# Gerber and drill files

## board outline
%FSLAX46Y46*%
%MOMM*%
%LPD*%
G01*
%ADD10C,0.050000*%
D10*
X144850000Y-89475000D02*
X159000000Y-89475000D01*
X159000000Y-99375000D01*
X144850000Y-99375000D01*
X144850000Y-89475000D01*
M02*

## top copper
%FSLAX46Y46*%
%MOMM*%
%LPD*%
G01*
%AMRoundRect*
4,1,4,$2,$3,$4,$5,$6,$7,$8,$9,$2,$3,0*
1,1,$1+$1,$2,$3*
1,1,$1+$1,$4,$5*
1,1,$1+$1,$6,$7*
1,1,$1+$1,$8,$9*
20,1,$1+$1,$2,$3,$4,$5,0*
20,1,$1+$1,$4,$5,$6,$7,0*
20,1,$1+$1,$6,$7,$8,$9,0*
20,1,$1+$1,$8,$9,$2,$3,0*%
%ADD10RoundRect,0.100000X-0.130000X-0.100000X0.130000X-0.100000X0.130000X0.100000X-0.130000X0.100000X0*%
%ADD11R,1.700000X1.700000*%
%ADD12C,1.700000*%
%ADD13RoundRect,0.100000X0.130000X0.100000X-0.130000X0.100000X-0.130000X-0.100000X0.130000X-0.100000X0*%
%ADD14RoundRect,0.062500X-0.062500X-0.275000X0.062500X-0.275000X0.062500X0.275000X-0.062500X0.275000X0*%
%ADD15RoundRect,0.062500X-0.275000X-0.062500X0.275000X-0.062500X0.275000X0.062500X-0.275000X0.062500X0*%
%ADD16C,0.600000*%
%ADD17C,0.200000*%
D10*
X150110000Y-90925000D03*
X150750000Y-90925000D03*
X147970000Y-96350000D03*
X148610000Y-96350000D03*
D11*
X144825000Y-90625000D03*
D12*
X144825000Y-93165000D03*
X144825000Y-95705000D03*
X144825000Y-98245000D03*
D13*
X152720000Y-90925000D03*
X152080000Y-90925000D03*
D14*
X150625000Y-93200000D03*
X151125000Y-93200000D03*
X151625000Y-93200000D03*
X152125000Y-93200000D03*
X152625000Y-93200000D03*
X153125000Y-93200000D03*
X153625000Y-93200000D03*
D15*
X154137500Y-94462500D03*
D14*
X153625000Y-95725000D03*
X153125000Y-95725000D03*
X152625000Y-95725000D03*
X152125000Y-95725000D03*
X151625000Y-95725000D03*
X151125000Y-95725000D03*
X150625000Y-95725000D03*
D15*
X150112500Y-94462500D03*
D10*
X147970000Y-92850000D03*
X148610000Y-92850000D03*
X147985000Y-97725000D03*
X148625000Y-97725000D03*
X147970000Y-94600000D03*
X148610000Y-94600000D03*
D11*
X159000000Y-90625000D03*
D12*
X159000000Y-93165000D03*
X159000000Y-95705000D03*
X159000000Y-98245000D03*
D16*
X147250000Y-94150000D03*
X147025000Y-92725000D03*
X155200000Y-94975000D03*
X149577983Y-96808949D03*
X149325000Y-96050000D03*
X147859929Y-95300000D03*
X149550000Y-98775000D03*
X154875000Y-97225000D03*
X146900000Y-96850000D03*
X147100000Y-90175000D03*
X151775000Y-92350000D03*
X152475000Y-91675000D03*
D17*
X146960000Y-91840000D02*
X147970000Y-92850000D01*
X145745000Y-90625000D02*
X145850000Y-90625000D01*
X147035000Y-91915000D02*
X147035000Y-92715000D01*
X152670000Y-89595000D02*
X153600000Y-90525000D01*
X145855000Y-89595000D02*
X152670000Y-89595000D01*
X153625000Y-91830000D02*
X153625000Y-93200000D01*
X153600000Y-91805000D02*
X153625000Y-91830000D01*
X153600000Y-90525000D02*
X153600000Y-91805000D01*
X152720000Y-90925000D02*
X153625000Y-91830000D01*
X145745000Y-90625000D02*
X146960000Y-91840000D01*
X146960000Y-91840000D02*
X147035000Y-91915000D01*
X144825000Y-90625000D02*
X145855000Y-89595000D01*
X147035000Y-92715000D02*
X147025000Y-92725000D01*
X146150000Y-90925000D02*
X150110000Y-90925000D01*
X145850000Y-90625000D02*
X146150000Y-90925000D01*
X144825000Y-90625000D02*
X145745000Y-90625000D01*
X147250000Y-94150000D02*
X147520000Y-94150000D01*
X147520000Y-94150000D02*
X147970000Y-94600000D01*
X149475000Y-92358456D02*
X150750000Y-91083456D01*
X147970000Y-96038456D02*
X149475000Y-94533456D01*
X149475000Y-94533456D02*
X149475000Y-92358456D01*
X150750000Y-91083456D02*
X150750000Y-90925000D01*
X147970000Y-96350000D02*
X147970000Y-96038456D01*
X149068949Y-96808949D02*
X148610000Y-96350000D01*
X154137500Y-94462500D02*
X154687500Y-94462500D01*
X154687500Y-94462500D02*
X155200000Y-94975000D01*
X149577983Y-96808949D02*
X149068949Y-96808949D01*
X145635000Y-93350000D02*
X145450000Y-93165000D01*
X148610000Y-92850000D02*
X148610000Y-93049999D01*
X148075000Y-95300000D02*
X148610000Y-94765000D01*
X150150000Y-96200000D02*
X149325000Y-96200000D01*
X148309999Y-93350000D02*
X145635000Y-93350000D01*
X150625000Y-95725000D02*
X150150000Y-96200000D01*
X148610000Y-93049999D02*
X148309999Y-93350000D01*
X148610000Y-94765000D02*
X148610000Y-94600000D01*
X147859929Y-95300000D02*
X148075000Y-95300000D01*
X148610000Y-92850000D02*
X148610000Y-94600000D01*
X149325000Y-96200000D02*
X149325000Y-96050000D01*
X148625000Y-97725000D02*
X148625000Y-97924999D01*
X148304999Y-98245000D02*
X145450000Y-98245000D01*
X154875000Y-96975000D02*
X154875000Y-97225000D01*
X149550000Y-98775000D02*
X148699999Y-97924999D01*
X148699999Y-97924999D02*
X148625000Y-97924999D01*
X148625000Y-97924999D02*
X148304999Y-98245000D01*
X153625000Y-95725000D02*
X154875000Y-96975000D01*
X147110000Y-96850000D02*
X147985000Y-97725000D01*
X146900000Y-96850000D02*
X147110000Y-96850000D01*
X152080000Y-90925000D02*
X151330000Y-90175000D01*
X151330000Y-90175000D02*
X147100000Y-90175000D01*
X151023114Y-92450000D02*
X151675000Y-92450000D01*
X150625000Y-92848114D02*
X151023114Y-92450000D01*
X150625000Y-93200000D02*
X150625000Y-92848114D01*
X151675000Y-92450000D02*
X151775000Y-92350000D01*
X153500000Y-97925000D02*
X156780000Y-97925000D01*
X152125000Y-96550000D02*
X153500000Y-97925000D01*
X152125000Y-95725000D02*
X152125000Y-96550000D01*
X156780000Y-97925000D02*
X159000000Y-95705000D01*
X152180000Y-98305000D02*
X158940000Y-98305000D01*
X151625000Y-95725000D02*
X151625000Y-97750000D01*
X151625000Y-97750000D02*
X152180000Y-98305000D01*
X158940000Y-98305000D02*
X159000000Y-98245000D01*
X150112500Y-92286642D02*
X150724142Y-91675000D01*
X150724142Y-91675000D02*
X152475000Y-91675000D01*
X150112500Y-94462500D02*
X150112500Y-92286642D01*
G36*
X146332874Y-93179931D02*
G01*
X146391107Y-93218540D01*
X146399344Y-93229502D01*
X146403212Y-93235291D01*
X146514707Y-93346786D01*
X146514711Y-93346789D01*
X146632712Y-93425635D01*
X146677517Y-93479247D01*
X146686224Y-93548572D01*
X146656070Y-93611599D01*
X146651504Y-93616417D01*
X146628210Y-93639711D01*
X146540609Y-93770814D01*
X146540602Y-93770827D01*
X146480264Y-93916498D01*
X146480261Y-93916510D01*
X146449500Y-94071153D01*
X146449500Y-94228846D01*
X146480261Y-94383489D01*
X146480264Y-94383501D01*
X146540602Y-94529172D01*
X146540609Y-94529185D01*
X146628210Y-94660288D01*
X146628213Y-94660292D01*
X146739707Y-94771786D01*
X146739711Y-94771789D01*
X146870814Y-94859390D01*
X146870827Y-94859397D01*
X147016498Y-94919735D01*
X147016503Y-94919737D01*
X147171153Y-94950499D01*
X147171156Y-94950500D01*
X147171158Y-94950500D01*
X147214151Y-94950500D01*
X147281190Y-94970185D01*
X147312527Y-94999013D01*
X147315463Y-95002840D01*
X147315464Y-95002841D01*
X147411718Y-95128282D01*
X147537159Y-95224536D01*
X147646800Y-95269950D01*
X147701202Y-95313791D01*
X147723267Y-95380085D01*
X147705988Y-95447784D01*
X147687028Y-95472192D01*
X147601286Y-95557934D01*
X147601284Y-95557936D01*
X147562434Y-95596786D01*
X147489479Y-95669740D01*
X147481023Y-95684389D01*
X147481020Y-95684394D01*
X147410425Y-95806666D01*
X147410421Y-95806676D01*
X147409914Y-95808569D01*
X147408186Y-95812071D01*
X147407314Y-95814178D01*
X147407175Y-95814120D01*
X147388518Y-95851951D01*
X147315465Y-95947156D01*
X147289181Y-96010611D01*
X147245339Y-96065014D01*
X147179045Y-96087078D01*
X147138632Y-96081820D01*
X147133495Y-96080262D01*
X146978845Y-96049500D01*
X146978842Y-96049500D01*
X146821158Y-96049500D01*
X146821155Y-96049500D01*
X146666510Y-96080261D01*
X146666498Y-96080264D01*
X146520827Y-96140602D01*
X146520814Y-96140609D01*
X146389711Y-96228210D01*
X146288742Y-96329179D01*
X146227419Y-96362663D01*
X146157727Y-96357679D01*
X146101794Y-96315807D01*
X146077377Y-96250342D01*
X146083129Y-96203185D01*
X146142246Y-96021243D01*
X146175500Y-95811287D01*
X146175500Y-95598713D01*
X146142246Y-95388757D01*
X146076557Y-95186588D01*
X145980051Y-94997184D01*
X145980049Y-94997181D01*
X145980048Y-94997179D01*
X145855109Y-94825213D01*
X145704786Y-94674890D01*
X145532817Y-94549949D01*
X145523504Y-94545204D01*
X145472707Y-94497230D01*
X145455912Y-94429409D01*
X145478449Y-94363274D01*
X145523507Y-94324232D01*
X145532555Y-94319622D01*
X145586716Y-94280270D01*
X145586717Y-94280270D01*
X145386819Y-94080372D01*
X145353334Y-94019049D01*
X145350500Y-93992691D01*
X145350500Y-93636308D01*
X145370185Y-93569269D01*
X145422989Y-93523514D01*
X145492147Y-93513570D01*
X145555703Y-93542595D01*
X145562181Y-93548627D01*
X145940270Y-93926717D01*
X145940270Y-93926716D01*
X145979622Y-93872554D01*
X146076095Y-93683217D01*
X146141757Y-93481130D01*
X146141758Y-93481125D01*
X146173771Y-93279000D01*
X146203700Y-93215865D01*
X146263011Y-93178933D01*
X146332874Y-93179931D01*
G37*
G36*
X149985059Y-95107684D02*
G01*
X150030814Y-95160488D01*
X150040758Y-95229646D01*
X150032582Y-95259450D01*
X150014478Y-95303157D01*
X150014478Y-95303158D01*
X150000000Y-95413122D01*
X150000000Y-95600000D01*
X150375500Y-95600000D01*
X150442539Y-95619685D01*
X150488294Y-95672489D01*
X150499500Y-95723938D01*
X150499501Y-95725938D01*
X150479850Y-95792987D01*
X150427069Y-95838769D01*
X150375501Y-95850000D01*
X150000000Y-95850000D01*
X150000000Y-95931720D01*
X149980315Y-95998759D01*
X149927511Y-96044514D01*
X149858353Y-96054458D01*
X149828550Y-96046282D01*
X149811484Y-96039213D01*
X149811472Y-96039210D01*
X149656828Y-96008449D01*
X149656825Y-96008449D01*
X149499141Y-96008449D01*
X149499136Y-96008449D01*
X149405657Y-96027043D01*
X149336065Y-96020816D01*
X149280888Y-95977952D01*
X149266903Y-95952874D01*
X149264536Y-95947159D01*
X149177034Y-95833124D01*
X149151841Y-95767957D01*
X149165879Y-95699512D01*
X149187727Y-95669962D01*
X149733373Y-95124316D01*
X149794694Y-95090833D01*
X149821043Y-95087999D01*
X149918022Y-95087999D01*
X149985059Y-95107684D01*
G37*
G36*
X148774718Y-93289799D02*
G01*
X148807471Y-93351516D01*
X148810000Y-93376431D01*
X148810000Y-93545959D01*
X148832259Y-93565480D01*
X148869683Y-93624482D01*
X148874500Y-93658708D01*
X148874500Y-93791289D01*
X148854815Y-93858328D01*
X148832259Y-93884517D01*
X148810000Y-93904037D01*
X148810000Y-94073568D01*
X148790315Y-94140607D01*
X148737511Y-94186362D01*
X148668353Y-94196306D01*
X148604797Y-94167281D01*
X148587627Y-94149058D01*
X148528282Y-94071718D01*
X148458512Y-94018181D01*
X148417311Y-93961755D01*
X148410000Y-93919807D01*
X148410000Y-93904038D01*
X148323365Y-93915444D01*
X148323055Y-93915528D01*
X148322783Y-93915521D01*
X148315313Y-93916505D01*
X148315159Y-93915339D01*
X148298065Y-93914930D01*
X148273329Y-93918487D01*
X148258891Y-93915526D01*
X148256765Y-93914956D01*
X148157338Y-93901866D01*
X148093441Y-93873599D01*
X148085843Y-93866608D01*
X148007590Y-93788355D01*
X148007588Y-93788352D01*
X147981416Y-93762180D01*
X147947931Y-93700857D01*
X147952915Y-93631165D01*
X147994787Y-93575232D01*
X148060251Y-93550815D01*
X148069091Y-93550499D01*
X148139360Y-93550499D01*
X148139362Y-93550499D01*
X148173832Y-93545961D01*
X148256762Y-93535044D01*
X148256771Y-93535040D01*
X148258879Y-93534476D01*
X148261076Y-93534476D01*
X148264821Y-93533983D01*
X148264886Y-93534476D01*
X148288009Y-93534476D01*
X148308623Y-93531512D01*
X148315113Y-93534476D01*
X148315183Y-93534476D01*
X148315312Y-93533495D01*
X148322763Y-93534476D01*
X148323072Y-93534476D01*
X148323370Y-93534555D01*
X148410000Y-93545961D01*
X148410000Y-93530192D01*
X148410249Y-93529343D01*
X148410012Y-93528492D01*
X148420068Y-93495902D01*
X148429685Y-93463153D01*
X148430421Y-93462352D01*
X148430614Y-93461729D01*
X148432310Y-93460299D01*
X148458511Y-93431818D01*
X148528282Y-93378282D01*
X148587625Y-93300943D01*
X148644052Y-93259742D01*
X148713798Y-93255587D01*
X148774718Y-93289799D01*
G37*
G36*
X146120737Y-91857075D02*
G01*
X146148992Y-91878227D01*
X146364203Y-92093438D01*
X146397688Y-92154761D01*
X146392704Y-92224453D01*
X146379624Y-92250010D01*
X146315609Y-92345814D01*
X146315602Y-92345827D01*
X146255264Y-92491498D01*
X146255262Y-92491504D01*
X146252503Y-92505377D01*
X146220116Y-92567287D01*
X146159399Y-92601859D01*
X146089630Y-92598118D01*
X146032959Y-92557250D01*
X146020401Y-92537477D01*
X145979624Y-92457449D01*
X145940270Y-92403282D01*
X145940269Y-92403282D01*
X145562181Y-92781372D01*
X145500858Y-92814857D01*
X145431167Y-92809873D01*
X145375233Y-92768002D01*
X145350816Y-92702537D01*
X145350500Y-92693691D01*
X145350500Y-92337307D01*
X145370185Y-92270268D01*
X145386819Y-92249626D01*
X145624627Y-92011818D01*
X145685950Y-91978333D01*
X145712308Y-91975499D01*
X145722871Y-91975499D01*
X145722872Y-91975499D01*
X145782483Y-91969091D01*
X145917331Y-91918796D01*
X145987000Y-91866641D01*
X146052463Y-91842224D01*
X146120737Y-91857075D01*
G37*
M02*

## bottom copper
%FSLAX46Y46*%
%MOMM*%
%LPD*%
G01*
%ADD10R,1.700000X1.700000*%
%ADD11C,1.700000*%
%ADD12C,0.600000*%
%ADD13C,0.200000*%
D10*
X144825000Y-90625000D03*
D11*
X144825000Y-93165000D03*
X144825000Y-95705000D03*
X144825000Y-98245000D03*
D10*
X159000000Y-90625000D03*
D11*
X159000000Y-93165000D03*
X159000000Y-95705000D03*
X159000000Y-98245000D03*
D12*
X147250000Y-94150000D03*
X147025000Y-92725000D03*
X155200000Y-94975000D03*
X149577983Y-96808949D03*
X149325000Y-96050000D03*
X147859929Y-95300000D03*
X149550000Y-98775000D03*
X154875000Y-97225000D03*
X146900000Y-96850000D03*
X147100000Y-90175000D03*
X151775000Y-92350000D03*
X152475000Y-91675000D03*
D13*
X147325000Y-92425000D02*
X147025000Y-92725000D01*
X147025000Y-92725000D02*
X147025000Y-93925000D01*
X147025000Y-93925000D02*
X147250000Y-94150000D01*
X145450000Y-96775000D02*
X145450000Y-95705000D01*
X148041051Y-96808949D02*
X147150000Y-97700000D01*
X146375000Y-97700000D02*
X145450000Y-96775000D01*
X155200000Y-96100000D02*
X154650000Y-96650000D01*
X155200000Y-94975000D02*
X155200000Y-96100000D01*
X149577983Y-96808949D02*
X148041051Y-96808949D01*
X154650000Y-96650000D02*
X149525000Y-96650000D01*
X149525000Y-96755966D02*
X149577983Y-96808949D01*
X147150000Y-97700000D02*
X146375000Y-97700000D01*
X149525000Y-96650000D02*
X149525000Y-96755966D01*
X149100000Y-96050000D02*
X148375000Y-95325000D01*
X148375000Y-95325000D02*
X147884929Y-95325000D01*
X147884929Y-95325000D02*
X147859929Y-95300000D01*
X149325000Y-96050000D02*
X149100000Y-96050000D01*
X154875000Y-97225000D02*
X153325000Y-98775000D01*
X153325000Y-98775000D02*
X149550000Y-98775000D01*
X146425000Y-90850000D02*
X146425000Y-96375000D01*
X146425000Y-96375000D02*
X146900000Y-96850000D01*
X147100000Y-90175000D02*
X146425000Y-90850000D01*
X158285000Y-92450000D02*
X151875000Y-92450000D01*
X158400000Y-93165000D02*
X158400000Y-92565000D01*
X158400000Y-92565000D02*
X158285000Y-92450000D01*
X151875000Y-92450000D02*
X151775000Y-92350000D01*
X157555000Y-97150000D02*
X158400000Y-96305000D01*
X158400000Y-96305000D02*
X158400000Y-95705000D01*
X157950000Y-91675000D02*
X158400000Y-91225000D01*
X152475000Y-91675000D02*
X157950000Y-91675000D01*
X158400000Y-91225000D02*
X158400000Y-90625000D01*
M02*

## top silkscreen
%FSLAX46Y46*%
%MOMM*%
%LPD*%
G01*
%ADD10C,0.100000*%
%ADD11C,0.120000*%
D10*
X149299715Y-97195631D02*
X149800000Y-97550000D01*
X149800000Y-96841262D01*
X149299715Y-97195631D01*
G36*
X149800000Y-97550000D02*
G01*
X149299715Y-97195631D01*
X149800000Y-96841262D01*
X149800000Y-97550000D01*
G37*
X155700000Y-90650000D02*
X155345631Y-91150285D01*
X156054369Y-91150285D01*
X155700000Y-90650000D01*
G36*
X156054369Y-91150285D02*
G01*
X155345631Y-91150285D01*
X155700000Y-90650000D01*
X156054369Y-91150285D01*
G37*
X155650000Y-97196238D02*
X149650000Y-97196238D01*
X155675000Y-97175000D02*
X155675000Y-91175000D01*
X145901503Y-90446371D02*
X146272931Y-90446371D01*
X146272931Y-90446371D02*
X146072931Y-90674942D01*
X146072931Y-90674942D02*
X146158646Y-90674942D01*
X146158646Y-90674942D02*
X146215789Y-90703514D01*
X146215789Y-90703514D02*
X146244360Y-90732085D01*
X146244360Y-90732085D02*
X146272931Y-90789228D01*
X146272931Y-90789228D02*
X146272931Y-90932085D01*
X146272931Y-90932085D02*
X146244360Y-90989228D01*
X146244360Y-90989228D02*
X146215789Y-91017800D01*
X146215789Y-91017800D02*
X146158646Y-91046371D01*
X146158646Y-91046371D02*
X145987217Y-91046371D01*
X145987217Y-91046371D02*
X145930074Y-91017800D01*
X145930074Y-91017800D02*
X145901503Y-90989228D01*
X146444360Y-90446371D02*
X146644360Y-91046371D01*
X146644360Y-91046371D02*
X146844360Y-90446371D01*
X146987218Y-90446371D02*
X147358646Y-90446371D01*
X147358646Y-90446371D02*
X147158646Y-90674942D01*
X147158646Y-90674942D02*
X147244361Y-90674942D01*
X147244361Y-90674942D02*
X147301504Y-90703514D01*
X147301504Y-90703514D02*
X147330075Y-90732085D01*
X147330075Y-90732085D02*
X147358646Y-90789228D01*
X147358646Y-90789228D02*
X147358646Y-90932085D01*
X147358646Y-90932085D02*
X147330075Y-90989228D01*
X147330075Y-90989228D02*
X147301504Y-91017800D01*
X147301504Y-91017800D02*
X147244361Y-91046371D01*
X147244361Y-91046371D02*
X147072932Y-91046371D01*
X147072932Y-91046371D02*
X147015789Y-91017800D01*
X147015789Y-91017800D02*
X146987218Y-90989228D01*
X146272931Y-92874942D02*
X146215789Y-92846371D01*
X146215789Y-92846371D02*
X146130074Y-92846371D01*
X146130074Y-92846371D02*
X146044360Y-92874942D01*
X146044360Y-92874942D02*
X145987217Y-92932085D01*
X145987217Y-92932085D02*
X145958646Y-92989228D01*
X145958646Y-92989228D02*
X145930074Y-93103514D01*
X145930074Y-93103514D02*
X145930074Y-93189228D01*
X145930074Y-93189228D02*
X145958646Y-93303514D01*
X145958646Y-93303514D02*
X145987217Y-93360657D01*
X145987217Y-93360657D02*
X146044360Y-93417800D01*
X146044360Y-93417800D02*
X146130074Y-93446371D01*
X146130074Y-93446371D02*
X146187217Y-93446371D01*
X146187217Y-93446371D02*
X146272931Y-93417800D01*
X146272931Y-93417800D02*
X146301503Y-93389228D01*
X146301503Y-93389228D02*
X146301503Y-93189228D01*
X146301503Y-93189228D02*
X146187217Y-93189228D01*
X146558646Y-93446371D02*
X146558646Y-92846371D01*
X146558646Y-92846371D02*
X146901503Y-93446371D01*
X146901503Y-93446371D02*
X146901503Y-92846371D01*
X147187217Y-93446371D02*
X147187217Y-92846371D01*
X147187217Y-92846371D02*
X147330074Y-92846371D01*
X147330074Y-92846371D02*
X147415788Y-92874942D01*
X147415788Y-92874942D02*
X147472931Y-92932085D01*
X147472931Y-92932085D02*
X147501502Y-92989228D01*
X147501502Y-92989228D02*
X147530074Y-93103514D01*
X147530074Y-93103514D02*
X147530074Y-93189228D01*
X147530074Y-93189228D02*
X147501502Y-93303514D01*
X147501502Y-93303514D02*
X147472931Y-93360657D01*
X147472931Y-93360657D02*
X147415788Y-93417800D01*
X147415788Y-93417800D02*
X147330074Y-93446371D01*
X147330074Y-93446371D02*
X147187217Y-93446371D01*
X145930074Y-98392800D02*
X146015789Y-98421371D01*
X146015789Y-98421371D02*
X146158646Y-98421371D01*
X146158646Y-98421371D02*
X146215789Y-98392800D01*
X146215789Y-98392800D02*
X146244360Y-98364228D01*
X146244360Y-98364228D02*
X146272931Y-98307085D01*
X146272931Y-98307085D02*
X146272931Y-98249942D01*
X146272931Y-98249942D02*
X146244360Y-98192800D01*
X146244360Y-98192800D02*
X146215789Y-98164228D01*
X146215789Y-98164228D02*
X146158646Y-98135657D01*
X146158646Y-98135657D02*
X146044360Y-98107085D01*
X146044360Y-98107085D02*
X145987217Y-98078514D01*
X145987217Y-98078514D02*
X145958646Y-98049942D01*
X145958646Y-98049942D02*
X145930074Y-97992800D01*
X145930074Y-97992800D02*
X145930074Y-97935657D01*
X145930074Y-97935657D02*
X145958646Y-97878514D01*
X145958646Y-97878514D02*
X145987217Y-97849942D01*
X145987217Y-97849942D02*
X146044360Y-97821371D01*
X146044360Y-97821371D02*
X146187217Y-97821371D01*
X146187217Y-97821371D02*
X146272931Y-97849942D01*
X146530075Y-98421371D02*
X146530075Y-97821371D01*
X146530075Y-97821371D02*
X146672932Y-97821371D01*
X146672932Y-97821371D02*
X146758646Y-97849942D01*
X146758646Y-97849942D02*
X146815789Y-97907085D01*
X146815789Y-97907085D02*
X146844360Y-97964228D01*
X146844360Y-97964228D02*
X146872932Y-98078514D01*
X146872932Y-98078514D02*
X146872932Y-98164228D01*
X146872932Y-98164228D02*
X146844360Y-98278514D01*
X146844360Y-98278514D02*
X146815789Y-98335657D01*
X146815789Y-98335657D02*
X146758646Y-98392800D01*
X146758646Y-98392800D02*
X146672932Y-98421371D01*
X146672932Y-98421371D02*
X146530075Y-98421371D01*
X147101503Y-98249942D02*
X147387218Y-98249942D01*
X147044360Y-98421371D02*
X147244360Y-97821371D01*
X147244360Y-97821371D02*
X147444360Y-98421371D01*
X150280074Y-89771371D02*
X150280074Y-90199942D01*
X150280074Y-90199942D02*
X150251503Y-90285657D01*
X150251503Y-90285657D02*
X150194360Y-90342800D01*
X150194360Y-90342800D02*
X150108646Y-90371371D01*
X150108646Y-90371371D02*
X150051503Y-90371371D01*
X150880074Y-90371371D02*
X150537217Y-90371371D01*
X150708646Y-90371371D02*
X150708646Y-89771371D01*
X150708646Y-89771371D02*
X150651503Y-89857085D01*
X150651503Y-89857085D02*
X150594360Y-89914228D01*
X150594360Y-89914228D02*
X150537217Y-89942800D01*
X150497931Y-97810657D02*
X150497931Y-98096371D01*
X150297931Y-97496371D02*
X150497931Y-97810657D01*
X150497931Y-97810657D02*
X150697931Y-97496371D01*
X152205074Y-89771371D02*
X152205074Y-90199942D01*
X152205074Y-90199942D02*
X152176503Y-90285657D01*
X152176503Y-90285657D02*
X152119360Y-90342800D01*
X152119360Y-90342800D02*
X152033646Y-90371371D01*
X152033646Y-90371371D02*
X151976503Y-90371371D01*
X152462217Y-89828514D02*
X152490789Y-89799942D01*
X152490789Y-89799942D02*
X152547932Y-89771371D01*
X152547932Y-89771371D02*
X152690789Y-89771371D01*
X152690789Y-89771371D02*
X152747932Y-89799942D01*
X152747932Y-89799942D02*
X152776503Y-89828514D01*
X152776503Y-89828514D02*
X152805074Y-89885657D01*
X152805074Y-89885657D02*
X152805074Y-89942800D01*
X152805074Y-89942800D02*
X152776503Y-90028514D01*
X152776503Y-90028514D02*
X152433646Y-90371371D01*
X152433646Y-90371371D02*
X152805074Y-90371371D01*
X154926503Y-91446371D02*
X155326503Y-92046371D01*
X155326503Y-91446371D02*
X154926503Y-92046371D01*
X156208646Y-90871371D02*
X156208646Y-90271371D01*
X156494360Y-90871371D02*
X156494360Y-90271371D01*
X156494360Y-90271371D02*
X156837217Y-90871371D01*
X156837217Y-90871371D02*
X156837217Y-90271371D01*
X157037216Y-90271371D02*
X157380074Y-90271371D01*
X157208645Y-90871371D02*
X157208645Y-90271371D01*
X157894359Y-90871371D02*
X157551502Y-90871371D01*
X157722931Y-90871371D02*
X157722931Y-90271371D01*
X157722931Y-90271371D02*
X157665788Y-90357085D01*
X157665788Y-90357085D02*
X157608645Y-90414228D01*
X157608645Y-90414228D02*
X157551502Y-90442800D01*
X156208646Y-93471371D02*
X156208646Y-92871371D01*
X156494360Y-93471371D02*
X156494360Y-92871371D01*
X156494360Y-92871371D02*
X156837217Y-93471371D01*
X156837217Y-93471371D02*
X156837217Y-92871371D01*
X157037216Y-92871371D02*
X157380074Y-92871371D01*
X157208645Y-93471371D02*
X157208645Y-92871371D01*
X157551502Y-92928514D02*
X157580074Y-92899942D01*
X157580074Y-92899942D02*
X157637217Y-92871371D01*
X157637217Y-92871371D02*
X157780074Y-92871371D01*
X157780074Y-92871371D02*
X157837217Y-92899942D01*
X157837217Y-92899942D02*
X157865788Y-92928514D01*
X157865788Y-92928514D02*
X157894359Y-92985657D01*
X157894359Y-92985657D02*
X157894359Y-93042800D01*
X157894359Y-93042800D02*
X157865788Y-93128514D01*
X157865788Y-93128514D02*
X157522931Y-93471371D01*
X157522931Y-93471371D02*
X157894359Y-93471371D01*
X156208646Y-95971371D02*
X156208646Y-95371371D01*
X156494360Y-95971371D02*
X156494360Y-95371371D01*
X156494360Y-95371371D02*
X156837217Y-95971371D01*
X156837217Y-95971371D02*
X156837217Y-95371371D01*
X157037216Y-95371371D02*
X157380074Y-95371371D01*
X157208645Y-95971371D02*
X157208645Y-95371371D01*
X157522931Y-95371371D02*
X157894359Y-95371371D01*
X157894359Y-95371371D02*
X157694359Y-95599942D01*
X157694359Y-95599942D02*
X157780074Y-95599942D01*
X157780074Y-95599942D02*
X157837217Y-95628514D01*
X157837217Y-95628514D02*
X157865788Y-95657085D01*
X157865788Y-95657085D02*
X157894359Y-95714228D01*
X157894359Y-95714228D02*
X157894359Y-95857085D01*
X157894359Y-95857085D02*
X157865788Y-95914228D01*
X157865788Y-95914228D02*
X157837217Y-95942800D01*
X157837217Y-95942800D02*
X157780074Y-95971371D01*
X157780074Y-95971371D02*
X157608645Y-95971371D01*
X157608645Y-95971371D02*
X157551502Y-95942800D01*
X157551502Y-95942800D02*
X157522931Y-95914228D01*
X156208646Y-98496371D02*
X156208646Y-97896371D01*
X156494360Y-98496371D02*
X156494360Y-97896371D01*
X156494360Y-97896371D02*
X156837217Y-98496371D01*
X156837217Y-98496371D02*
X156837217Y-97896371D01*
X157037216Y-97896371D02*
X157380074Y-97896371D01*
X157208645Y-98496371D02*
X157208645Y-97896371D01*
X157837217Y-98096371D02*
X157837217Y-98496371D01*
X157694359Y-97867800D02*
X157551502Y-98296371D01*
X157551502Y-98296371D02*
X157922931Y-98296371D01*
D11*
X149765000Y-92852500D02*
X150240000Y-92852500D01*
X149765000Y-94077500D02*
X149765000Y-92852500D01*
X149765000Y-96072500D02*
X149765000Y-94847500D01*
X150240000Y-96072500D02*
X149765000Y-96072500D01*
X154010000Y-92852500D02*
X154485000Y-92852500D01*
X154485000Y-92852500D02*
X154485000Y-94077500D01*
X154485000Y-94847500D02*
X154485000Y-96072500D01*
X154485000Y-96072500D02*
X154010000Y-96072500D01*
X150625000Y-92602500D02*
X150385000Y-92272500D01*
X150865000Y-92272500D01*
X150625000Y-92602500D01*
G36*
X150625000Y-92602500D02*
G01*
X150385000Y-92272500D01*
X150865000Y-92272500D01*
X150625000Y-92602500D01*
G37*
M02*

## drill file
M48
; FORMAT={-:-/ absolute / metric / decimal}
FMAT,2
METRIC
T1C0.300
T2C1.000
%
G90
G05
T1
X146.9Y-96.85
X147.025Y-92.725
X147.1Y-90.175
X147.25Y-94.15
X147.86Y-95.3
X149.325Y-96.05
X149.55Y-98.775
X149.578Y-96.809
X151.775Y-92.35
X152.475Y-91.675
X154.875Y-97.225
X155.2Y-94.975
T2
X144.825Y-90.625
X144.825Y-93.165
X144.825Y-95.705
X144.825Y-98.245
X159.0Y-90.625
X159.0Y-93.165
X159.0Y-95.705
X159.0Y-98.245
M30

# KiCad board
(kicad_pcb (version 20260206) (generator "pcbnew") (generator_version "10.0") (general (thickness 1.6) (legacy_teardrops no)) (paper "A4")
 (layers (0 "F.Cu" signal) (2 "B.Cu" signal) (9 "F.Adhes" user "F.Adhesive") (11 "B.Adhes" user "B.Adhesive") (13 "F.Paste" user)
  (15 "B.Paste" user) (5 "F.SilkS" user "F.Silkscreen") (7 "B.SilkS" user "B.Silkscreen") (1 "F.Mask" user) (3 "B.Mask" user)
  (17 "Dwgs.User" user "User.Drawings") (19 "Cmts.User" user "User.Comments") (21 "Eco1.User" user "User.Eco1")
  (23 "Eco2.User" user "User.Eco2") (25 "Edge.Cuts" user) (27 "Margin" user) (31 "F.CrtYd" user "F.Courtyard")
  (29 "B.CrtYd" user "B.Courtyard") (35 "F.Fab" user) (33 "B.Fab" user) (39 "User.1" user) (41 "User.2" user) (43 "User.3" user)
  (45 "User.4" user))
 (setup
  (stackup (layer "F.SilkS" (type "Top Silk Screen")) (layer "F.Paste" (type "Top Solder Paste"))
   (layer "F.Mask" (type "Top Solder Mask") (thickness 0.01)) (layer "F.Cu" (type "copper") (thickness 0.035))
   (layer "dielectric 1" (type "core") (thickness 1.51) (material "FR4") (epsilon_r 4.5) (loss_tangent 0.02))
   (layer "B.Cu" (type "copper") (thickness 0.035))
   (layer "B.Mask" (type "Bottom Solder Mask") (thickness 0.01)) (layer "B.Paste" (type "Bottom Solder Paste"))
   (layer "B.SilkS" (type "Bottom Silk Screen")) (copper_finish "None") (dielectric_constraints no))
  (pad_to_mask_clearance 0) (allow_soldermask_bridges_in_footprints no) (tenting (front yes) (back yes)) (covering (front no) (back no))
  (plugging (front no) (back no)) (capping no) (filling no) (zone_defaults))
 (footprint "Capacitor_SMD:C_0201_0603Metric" (layer "F.Cu") (at 150.43 90.925)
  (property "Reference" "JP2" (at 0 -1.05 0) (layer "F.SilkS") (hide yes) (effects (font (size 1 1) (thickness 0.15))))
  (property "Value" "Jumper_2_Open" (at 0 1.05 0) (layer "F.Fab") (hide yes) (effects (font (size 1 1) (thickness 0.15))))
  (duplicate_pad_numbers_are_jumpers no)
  (pad "" smd roundrect (at -0.345 0) (size 0.318 0.36) (layers "F.Paste") (roundrect_rratio 0.25))
  (pad "" smd roundrect (at 0.345 0) (size 0.318 0.36) (layers "F.Paste") (roundrect_rratio 0.25))
  (pad "1" smd roundrect (at -0.32 0) (size 0.46 0.4) (layers "F.Cu" "F.Mask") (roundrect_rratio 0.25) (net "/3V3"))
  (pad "2" smd roundrect (at 0.32 0) (size 0.46 0.4) (layers "F.Cu" "F.Mask") (roundrect_rratio 0.25) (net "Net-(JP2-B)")))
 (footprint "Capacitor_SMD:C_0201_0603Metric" (layer "F.Cu") (at 148.29 96.35)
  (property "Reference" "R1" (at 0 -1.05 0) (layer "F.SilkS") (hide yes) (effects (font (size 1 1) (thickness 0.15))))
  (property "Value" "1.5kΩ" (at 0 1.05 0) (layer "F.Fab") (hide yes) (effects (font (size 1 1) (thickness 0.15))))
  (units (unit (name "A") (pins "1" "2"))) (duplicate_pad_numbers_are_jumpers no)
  (pad "" smd roundrect (at -0.345 0) (size 0.318 0.36) (layers "F.Paste") (roundrect_rratio 0.25))
  (pad "" smd roundrect (at 0.345 0) (size 0.318 0.36) (layers "F.Paste") (roundrect_rratio 0.25))
  (pad "1" smd roundrect (at -0.32 0) (size 0.46 0.4) (layers "F.Cu" "F.Mask") (roundrect_rratio 0.25) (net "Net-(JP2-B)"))
  (pad "2" smd roundrect (at 0.32 0) (size 0.46 0.4) (layers "F.Cu" "F.Mask") (roundrect_rratio 0.25) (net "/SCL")))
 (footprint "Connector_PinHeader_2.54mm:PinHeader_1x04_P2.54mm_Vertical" (layer "F.Cu") (at 144.825 90.625)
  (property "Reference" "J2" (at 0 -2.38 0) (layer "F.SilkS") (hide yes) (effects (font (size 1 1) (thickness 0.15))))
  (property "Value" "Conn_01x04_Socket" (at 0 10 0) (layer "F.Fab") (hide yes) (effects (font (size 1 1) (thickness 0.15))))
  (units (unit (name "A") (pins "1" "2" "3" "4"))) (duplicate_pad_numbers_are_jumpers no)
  (pad "1" thru_hole rect (at 0 0) (size 1.7 1.7) (drill 1) (layers "*.Cu" "*.Mask") (remove_unused_layers no) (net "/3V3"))
  (pad "2" thru_hole circle (at 0 2.54) (size 1.7 1.7) (drill 1) (layers "*.Cu" "*.Mask") (remove_unused_layers no) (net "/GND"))
  (pad "3" thru_hole circle (at 0 5.08) (size 1.7 1.7) (drill 1) (layers "*.Cu" "*.Mask") (remove_unused_layers no) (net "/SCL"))
  (pad "4" thru_hole circle (at 0 7.62) (size 1.7 1.7) (drill 1) (layers "*.Cu" "*.Mask") (remove_unused_layers no) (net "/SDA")))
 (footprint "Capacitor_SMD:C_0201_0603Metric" (layer "F.Cu") (at 152.4 90.925 180)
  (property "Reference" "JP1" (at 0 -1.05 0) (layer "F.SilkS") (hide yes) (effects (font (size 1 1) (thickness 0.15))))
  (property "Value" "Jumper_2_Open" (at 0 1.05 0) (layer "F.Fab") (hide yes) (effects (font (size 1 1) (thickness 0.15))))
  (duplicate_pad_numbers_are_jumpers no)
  (pad "" smd roundrect (at -0.345 0 180) (size 0.318 0.36) (layers "F.Paste") (roundrect_rratio 0.25))
  (pad "" smd roundrect (at 0.345 0 180) (size 0.318 0.36) (layers "F.Paste") (roundrect_rratio 0.25))
  (pad "1" smd roundrect (at -0.32 0 180) (size 0.46 0.4) (layers "F.Cu" "F.Mask") (roundrect_rratio 0.25) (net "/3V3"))
  (pad "2" smd roundrect (at 0.32 0 180) (size 0.46 0.4) (layers "F.Cu" "F.Mask") (roundrect_rratio 0.25) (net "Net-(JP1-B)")))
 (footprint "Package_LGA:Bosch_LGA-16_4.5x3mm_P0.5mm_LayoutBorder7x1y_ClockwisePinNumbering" (layer "F.Cu") (at 152.125 94.4625)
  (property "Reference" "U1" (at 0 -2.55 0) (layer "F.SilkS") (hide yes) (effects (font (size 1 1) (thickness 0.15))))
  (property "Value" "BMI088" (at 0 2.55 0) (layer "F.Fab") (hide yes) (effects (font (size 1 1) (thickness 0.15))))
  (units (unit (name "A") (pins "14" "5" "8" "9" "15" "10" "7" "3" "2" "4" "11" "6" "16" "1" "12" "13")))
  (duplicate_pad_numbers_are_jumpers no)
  (fp_line (start -2.36 -1.61) (end -1.885 -1.61) (stroke (width 0.12) (type solid)) (layer "F.SilkS"))
  (fp_line (start -2.36 -0.385) (end -2.36 -1.61) (stroke (width 0.12) (type solid)) (layer "F.SilkS"))
  (fp_line (start -2.36 1.61) (end -2.36 0.385) (stroke (width 0.12) (type solid)) (layer "F.SilkS"))
  (fp_line (start -1.885 1.61) (end -2.36 1.61) (stroke (width 0.12) (type solid)) (layer "F.SilkS"))
  (fp_line (start 1.885 -1.61) (end 2.36 -1.61) (stroke (width 0.12) (type solid)) (layer "F.SilkS"))
  (fp_line (start 2.36 -1.61) (end 2.36 -0.385) (stroke (width 0.12) (type solid)) (layer "F.SilkS"))
  (fp_line (start 2.36 0.385) (end 2.36 1.61) (stroke (width 0.12) (type solid)) (layer "F.SilkS"))
  (fp_line (start 2.36 1.61) (end 1.885 1.61) (stroke (width 0.12) (type solid)) (layer "F.SilkS"))
  (fp_poly (pts (xy -1.5 -1.86) (xy -1.74 -2.19) (xy -1.26 -2.19)) (stroke (width 0.12) (type solid)) (fill yes) (layer "F.SilkS"))
  (pad "1" smd roundrect (at -1.5 -1.2625) (size 0.25 0.675) (layers "F.Cu" "F.Mask" "F.Paste") (roundrect_rratio 0.25) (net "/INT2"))
  (pad "2" smd roundrect (at -1 -1.2625) (size 0.25 0.675) (layers "F.Cu" "F.Mask" "F.Paste") (roundrect_rratio 0.25) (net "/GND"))
  (pad "3" smd roundrect (at -0.5 -1.2625) (size 0.25 0.675) (layers "F.Cu" "F.Mask" "F.Paste") (roundrect_rratio 0.25) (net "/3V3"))
  (pad "4" smd roundrect (at 0 -1.2625) (size 0.25 0.675) (layers "F.Cu" "F.Mask" "F.Paste") (roundrect_rratio 0.25) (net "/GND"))
  (pad "5" smd roundrect (at 0.5 -1.2625) (size 0.25 0.675) (layers "F.Cu" "F.Mask" "F.Paste") (roundrect_rratio 0.25)
   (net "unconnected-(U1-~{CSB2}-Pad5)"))
  (pad "6" smd roundrect (at 1 -1.2625) (size 0.25 0.675) (layers "F.Cu" "F.Mask" "F.Paste") (roundrect_rratio 0.25) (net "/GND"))
  (pad "7" smd roundrect (at 1.5 -1.2625) (size 0.25 0.675) (layers "F.Cu" "F.Mask" "F.Paste") (roundrect_rratio 0.25) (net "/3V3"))
  (pad "8" smd roundrect (at 2.0125 0) (size 0.675 0.25) (layers "F.Cu" "F.Mask" "F.Paste") (roundrect_rratio 0.25) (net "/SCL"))
  (pad "9" smd roundrect (at 1.5 1.2625) (size 0.25 0.675) (layers "F.Cu" "F.Mask" "F.Paste") (roundrect_rratio 0.25) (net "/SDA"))
  (pad "10" smd roundrect (at 1 1.2625) (size 0.25 0.675) (layers "F.Cu" "F.Mask" "F.Paste") (roundrect_rratio 0.25) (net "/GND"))
  (pad "11" smd roundrect (at 0.5 1.2625) (size 0.25 0.675) (layers "F.Cu" "F.Mask" "F.Paste") (roundrect_rratio 0.25) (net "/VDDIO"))
  (pad "12" smd roundrect (at 0 1.2625) (size 0.25 0.675) (layers "F.Cu" "F.Mask" "F.Paste") (roundrect_rratio 0.25) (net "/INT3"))
  (pad "13" smd roundrect (at -0.5 1.2625) (size 0.25 0.675) (layers "F.Cu" "F.Mask" "F.Paste") (roundrect_rratio 0.25) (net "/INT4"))
  (pad "14" smd roundrect (at -1 1.2625) (size 0.25 0.675) (layers "F.Cu" "F.Mask" "F.Paste") (roundrect_rratio 0.25)
   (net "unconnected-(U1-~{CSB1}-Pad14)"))
  (pad "15" smd roundrect (at -1.5 1.2625) (size 0.25 0.675) (layers "F.Cu" "F.Mask" "F.Paste") (roundrect_rratio 0.25) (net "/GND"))
  (pad "16" smd roundrect (at -2.0125 0) (size 0.675 0.25) (layers "F.Cu" "F.Mask" "F.Paste") (roundrect_rratio 0.25) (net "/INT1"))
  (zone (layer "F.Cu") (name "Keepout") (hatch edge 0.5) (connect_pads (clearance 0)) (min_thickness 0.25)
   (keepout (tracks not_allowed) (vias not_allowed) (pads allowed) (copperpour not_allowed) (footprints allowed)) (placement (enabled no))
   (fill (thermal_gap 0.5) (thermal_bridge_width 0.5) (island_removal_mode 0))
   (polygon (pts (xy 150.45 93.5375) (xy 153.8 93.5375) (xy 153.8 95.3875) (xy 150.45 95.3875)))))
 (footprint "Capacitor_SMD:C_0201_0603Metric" (layer "F.Cu") (at 148.29 92.85)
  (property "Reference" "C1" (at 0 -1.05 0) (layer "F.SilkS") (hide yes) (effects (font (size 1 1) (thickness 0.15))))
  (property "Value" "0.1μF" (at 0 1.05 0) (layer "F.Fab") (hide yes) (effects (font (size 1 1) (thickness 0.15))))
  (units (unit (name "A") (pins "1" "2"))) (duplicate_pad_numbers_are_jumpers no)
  (pad "" smd roundrect (at -0.345 0) (size 0.318 0.36) (layers "F.Paste") (roundrect_rratio 0.25))
  (pad "" smd roundrect (at 0.345 0) (size 0.318 0.36) (layers "F.Paste") (roundrect_rratio 0.25))
  (pad "1" smd roundrect (at -0.32 0) (size 0.46 0.4) (layers "F.Cu" "F.Mask") (roundrect_rratio 0.25) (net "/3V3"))
  (pad "2" smd roundrect (at 0.32 0) (size 0.46 0.4) (layers "F.Cu" "F.Mask") (roundrect_rratio 0.25) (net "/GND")))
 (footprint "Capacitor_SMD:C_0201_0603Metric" (layer "F.Cu") (at 148.305 97.725)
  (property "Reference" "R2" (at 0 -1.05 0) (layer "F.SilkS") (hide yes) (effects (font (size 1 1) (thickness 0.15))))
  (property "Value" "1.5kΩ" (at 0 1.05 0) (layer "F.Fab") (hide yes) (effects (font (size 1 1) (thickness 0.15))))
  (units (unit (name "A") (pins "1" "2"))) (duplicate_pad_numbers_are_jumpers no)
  (pad "" smd roundrect (at -0.345 0) (size 0.318 0.36) (layers "F.Paste") (roundrect_rratio 0.25))
  (pad "" smd roundrect (at 0.345 0) (size 0.318 0.36) (layers "F.Paste") (roundrect_rratio 0.25))
  (pad "1" smd roundrect (at -0.32 0) (size 0.46 0.4) (layers "F.Cu" "F.Mask") (roundrect_rratio 0.25) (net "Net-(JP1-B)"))
  (pad "2" smd roundrect (at 0.32 0) (size 0.46 0.4) (layers "F.Cu" "F.Mask") (roundrect_rratio 0.25) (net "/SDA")))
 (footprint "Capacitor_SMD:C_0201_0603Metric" (layer "F.Cu") (at 148.29 94.6)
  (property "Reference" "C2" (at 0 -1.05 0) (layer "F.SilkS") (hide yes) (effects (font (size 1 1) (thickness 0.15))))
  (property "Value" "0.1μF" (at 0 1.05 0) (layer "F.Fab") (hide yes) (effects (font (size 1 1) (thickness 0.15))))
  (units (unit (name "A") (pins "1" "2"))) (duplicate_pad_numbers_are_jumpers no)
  (pad "" smd roundrect (at -0.345 0) (size 0.318 0.36) (layers "F.Paste") (roundrect_rratio 0.25))
  (pad "" smd roundrect (at 0.345 0) (size 0.318 0.36) (layers "F.Paste") (roundrect_rratio 0.25))
  (pad "1" smd roundrect (at -0.32 0) (size 0.46 0.4) (layers "F.Cu" "F.Mask") (roundrect_rratio 0.25) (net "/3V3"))
  (pad "2" smd roundrect (at 0.32 0) (size 0.46 0.4) (layers "F.Cu" "F.Mask") (roundrect_rratio 0.25) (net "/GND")))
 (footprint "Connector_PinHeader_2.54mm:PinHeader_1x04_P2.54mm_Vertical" (layer "F.Cu") (at 159 90.625)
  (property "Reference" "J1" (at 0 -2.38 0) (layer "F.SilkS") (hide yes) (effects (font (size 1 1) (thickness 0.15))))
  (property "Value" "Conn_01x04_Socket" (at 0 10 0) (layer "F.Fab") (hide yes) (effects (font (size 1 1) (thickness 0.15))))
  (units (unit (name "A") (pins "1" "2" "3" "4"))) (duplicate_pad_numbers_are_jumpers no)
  (pad "1" thru_hole rect (at 0 0) (size 1.7 1.7) (drill 1) (layers "*.Cu" "*.Mask") (remove_unused_layers no) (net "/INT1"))
  (pad "2" thru_hole circle (at 0 2.54) (size 1.7 1.7) (drill 1) (layers "*.Cu" "*.Mask") (remove_unused_layers no) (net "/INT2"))
  (pad "3" thru_hole circle (at 0 5.08) (size 1.7 1.7) (drill 1) (layers "*.Cu" "*.Mask") (remove_unused_layers no) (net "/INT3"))
  (pad "4" thru_hole circle (at 0 7.62) (size 1.7 1.7) (drill 1) (layers "*.Cu" "*.Mask") (remove_unused_layers no) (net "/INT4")))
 (gr_poly
  (pts (xy 149.299715 97.195631) (xy 149.8 97.55) (xy 149.8 96.841262)) (stroke (width 0.1) (type solid)) (fill yes) (layer "F.SilkS"))
 (gr_poly
  (pts (xy 155.7 90.65) (xy 155.345631 91.150285) (xy 156.054369 91.150285)) (stroke (width 0.1) (type solid)) (fill yes) (layer "F.SilkS"))
 (gr_line (start 155.65 97.196238) (end 149.65 97.196238) (stroke (width 0.1) (type solid)) (layer "F.SilkS"))
 (gr_line (start 155.675 97.175) (end 155.675 91.175) (stroke (width 0.1) (type solid)) (layer "F.SilkS"))
 (gr_rect (start 144.85 89.475) (end 159 99.375) (stroke (width 0.05) (type solid)) (fill no) (layer "Edge.Cuts"))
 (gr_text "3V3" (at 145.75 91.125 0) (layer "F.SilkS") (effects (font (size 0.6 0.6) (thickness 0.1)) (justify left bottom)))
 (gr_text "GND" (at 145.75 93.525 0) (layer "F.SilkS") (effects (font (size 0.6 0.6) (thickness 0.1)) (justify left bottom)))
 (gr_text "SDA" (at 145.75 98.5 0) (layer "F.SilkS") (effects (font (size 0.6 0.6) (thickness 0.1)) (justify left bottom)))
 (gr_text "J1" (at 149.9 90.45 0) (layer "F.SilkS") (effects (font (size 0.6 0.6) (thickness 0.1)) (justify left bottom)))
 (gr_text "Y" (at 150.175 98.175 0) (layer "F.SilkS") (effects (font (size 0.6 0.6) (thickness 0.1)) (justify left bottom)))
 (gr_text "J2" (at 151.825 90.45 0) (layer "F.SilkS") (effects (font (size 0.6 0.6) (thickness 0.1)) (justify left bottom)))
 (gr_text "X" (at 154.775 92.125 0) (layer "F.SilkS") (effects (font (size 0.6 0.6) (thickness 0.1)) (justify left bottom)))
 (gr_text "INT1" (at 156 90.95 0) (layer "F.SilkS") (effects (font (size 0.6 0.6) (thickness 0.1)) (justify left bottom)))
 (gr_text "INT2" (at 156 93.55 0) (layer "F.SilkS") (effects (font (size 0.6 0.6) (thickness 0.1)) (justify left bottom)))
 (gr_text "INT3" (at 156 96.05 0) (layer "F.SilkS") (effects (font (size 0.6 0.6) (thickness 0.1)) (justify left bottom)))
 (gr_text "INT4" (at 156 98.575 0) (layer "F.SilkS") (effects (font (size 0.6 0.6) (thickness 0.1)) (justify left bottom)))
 (segment (start 146.96 91.84) (end 147.97 92.85) (width 0.2) (layer "F.Cu") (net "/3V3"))
 (segment (start 145.745 90.625) (end 145.85 90.625) (width 0.2) (layer "F.Cu") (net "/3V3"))
 (segment (start 147.035 91.915) (end 147.035 92.715) (width 0.2) (layer "F.Cu") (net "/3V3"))
 (segment (start 152.67 89.595) (end 153.6 90.525) (width 0.2) (layer "F.Cu") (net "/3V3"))
 (segment (start 145.855 89.595) (end 152.67 89.595) (width 0.2) (layer "F.Cu") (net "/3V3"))
 (segment (start 153.625 91.83) (end 153.625 93.2) (width 0.2) (layer "F.Cu") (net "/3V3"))
 (segment (start 153.6 91.805) (end 153.625 91.83) (width 0.2) (layer "F.Cu") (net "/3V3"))
 (segment (start 153.6 90.525) (end 153.6 91.805) (width 0.2) (layer "F.Cu") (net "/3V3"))
 (segment (start 152.72 90.925) (end 153.625 91.83) (width 0.2) (layer "F.Cu") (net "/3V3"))
 (segment (start 145.745 90.625) (end 146.96 91.84) (width 0.2) (layer "F.Cu") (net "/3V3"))
 (segment (start 146.96 91.84) (end 147.035 91.915) (width 0.2) (layer "F.Cu") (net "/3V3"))
 (segment (start 144.825 90.625) (end 145.855 89.595) (width 0.2) (layer "F.Cu") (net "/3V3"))
 (segment (start 147.035 92.715) (end 147.025 92.725) (width 0.2) (layer "F.Cu") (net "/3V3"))
 (segment (start 146.15 90.925) (end 150.11 90.925) (width 0.2) (layer "F.Cu") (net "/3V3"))
 (segment (start 145.85 90.625) (end 146.15 90.925) (width 0.2) (layer "F.Cu") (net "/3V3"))
 (segment (start 144.825 90.625) (end 145.745 90.625) (width 0.2) (layer "F.Cu") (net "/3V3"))
 (segment (start 147.25 94.15) (end 147.52 94.15) (width 0.2) (layer "F.Cu") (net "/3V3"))
 (segment (start 147.52 94.15) (end 147.97 94.6) (width 0.2) (layer "F.Cu") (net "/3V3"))
 (via (at 147.25 94.15) (size 0.6) (drill 0.3) (layers "F.Cu" "B.Cu") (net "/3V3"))
 (via (at 147.025 92.725) (size 0.6) (drill 0.3) (layers "F.Cu" "B.Cu") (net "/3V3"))
 (segment (start 147.325 92.425) (end 147.025 92.725) (width 0.2) (layer "B.Cu") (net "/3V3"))
 (segment (start 147.025 92.725) (end 147.025 93.925) (width 0.2) (layer "B.Cu") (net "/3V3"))
 (segment (start 147.025 93.925) (end 147.25 94.15) (width 0.2) (layer "B.Cu") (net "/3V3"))
 (segment (start 149.475 92.358456) (end 150.75 91.083456) (width 0.2) (layer "F.Cu") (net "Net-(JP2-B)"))
 (segment (start 147.97 96.038456) (end 149.475 94.533456) (width 0.2) (layer "F.Cu") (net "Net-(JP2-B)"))
 (segment (start 149.475 94.533456) (end 149.475 92.358456) (width 0.2) (layer "F.Cu") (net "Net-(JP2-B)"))
 (segment (start 150.75 91.083456) (end 150.75 90.925) (width 0.2) (layer "F.Cu") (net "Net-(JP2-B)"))
 (segment (start 147.97 96.35) (end 147.97 96.038456) (width 0.2) (layer "F.Cu") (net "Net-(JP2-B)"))
 (segment (start 149.068949 96.808949) (end 148.61 96.35) (width 0.2) (layer "F.Cu") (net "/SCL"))
 (segment (start 154.1375 94.4625) (end 154.6875 94.4625) (width 0.2) (layer "F.Cu") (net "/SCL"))
 (segment (start 154.6875 94.4625) (end 155.2 94.975) (width 0.2) (layer "F.Cu") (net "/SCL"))
 (segment (start 149.577983 96.808949) (end 149.068949 96.808949) (width 0.2) (layer "F.Cu") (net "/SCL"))
 (via (at 155.2 94.975) (size 0.6) (drill 0.3) (layers "F.Cu" "B.Cu") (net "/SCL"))
 (via (at 149.577983 96.808949) (size 0.6) (drill 0.3) (layers "F.Cu" "B.Cu") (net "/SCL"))
 (segment (start 145.45 96.775) (end 145.45 95.705) (width 0.2) (layer "B.Cu") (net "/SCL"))
 (segment (start 148.041051 96.808949) (end 147.15 97.7) (width 0.2) (layer "B.Cu") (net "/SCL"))
 (segment (start 146.375 97.7) (end 145.45 96.775) (width 0.2) (layer "B.Cu") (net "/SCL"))
 (segment (start 155.2 96.1) (end 154.65 96.65) (width 0.2) (layer "B.Cu") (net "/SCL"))
 (segment (start 155.2 94.975) (end 155.2 96.1) (width 0.2) (layer "B.Cu") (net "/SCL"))
 (segment (start 149.577983 96.808949) (end 148.041051 96.808949) (width 0.2) (layer "B.Cu") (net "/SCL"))
 (segment (start 154.65 96.65) (end 149.525 96.65) (width 0.2) (layer "B.Cu") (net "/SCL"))
 (segment (start 149.525 96.755966) (end 149.577983 96.808949) (width 0.2) (layer "B.Cu") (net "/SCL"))
 (segment (start 147.15 97.7) (end 146.375 97.7) (width 0.2) (layer "B.Cu") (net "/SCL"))
 (segment (start 149.525 96.65) (end 149.525 96.755966) (width 0.2) (layer "B.Cu") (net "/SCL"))
 (segment (start 145.635 93.35) (end 145.45 93.165) (width 0.2) (layer "F.Cu") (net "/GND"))
 (segment (start 148.61 92.85) (end 148.61 93.049999) (width 0.2) (layer "F.Cu") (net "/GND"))
 (segment (start 148.075 95.3) (end 148.61 94.765) (width 0.2) (layer "F.Cu") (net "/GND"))
 (segment (start 150.15 96.2) (end 149.325 96.2) (width 0.2) (layer "F.Cu") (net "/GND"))
 (segment (start 148.309999 93.35) (end 145.635 93.35) (width 0.2) (layer "F.Cu") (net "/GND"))
 (segment (start 150.625 95.725) (end 150.15 96.2) (width 0.2) (layer "F.Cu") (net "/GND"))
 (segment (start 148.61 93.049999) (end 148.309999 93.35) (width 0.2) (layer "F.Cu") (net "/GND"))
 (segment (start 148.61 94.765) (end 148.61 94.6) (width 0.2) (layer "F.Cu") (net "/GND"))
 (segment (start 147.859929 95.3) (end 148.075 95.3) (width 0.2) (layer "F.Cu") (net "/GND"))
 (segment (start 148.61 92.85) (end 148.61 94.6) (width 0.2) (layer "F.Cu") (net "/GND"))
 (segment (start 149.325 96.2) (end 149.325 96.05) (width 0.2) (layer "F.Cu") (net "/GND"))
 (via (at 149.325 96.05) (size 0.6) (drill 0.3) (layers "F.Cu" "B.Cu") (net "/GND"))
 (via (at 147.859929 95.3) (size 0.6) (drill 0.3) (layers "F.Cu" "B.Cu") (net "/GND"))
 (segment (start 149.1 96.05) (end 148.375 95.325) (width 0.2) (layer "B.Cu") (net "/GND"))
 (segment (start 148.375 95.325) (end 147.884929 95.325) (width 0.2) (layer "B.Cu") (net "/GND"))
 (segment (start 147.884929 95.325) (end 147.859929 95.3) (width 0.2) (layer "B.Cu") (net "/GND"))
 (segment (start 149.325 96.05) (end 149.1 96.05) (width 0.2) (layer "B.Cu") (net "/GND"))
 (segment (start 148.625 97.725) (end 148.625 97.924999) (width 0.2) (layer "F.Cu") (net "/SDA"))
 (segment (start 148.304999 98.245) (end 145.45 98.245) (width 0.2) (layer "F.Cu") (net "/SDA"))
 (segment (start 154.875 96.975) (end 154.875 97.225) (width 0.2) (layer "F.Cu") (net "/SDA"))
 (segment (start 149.55 98.775) (end 148.699999 97.924999) (width 0.2) (layer "F.Cu") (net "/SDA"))
 (segment (start 148.699999 97.924999) (end 148.625 97.924999) (width 0.2) (layer "F.Cu") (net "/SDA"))
 (segment (start 148.625 97.924999) (end 148.304999 98.245) (width 0.2) (layer "F.Cu") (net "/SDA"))
 (segment (start 153.625 95.725) (end 154.875 96.975) (width 0.2) (layer "F.Cu") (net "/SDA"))
 (via (at 149.55 98.775) (size 0.6) (drill 0.3) (layers "F.Cu" "B.Cu") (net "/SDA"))
 (via (at 154.875 97.225) (size 0.6) (drill 0.3) (layers "F.Cu" "B.Cu") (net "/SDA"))
 (segment (start 154.875 97.225) (end 153.325 98.775) (width 0.2) (layer "B.Cu") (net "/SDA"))
 (segment (start 153.325 98.775) (end 149.55 98.775) (width 0.2) (layer "B.Cu") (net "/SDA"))
 (segment (start 147.11 96.85) (end 147.985 97.725) (width 0.2) (layer "F.Cu") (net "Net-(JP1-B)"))
 (segment (start 146.9 96.85) (end 147.11 96.85) (width 0.2) (layer "F.Cu") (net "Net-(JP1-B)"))
 (segment (start 152.08 90.925) (end 151.33 90.175) (width 0.2) (layer "F.Cu") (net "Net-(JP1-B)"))
 (segment (start 151.33 90.175) (end 147.1 90.175) (width 0.2) (layer "F.Cu") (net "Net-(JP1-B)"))
 (via (at 146.9 96.85) (size 0.6) (drill 0.3) (layers "F.Cu" "B.Cu") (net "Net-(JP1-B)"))
 (via (at 147.1 90.175) (size 0.6) (drill 0.3) (layers "F.Cu" "B.Cu") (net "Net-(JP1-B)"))
 (segment (start 146.425 90.85) (end 146.425 96.375) (width 0.2) (layer "B.Cu") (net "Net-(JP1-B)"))
 (segment (start 146.425 96.375) (end 146.9 96.85) (width 0.2) (layer "B.Cu") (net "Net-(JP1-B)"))
 (segment (start 147.1 90.175) (end 146.425 90.85) (width 0.2) (layer "B.Cu") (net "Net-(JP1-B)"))
 (segment (start 151.023114 92.45) (end 151.675 92.45) (width 0.2) (layer "F.Cu") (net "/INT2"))
 (segment (start 150.625 92.848114) (end 151.023114 92.45) (width 0.2) (layer "F.Cu") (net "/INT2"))
 (segment (start 150.625 93.2) (end 150.625 92.848114) (width 0.2) (layer "F.Cu") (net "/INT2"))
 (segment (start 151.675 92.45) (end 151.775 92.35) (width 0.2) (layer "F.Cu") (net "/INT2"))
 (via (at 151.775 92.35) (size 0.6) (drill 0.3) (layers "F.Cu" "B.Cu") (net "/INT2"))
 (segment (start 158.285 92.45) (end 151.875 92.45) (width 0.2) (layer "B.Cu") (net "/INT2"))
 (segment (start 158.4 93.165) (end 158.4 92.565) (width 0.2) (layer "B.Cu") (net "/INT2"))
 (segment (start 158.4 92.565) (end 158.285 92.45) (width 0.2) (layer "B.Cu") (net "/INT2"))
 (segment (start 151.875 92.45) (end 151.775 92.35) (width 0.2) (layer "B.Cu") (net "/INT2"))
 (segment (start 153.5 97.925) (end 156.78 97.925) (width 0.2) (layer "F.Cu") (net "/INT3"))
 (segment (start 152.125 96.55) (end 153.5 97.925) (width 0.2) (layer "F.Cu") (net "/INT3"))
 (segment (start 152.125 95.725) (end 152.125 96.55) (width 0.2) (layer "F.Cu") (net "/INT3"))
 (segment (start 156.78 97.925) (end 159 95.705) (width 0.2) (layer "F.Cu") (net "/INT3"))
 (segment (start 157.555 97.15) (end 158.4 96.305) (width 0.2) (layer "B.Cu") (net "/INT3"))
 (segment (start 158.4 96.305) (end 158.4 95.705) (width 0.2) (layer "B.Cu") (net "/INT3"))
 (segment (start 152.18 98.305) (end 158.94 98.305) (width 0.2) (layer "F.Cu") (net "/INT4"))
 (segment (start 151.625 95.725) (end 151.625 97.75) (width 0.2) (layer "F.Cu") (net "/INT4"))
 (segment (start 151.625 97.75) (end 152.18 98.305) (width 0.2) (layer "F.Cu") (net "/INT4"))
 (segment (start 158.94 98.305) (end 159 98.245) (width 0.2) (layer "F.Cu") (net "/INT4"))
 (segment (start 150.1125 92.286642) (end 150.724142 91.675) (width 0.2) (layer "F.Cu") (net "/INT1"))
 (segment (start 150.724142 91.675) (end 152.475 91.675) (width 0.2) (layer "F.Cu") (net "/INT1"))
 (segment (start 150.1125 94.4625) (end 150.1125 92.286642) (width 0.2) (layer "F.Cu") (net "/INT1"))
 (via (at 152.475 91.675) (size 0.6) (drill 0.3) (layers "F.Cu" "B.Cu") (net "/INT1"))
 (segment (start 157.95 91.675) (end 158.4 91.225) (width 0.2) (layer "B.Cu") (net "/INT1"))
 (segment (start 152.475 91.675) (end 157.95 91.675) (width 0.2) (layer "B.Cu") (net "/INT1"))
 (segment (start 158.4 91.225) (end 158.4 90.625) (width 0.2) (layer "B.Cu") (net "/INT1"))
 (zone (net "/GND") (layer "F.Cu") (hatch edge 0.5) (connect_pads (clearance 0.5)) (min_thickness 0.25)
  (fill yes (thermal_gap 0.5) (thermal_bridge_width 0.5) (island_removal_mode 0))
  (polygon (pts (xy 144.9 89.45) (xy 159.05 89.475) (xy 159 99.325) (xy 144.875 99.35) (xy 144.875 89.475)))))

